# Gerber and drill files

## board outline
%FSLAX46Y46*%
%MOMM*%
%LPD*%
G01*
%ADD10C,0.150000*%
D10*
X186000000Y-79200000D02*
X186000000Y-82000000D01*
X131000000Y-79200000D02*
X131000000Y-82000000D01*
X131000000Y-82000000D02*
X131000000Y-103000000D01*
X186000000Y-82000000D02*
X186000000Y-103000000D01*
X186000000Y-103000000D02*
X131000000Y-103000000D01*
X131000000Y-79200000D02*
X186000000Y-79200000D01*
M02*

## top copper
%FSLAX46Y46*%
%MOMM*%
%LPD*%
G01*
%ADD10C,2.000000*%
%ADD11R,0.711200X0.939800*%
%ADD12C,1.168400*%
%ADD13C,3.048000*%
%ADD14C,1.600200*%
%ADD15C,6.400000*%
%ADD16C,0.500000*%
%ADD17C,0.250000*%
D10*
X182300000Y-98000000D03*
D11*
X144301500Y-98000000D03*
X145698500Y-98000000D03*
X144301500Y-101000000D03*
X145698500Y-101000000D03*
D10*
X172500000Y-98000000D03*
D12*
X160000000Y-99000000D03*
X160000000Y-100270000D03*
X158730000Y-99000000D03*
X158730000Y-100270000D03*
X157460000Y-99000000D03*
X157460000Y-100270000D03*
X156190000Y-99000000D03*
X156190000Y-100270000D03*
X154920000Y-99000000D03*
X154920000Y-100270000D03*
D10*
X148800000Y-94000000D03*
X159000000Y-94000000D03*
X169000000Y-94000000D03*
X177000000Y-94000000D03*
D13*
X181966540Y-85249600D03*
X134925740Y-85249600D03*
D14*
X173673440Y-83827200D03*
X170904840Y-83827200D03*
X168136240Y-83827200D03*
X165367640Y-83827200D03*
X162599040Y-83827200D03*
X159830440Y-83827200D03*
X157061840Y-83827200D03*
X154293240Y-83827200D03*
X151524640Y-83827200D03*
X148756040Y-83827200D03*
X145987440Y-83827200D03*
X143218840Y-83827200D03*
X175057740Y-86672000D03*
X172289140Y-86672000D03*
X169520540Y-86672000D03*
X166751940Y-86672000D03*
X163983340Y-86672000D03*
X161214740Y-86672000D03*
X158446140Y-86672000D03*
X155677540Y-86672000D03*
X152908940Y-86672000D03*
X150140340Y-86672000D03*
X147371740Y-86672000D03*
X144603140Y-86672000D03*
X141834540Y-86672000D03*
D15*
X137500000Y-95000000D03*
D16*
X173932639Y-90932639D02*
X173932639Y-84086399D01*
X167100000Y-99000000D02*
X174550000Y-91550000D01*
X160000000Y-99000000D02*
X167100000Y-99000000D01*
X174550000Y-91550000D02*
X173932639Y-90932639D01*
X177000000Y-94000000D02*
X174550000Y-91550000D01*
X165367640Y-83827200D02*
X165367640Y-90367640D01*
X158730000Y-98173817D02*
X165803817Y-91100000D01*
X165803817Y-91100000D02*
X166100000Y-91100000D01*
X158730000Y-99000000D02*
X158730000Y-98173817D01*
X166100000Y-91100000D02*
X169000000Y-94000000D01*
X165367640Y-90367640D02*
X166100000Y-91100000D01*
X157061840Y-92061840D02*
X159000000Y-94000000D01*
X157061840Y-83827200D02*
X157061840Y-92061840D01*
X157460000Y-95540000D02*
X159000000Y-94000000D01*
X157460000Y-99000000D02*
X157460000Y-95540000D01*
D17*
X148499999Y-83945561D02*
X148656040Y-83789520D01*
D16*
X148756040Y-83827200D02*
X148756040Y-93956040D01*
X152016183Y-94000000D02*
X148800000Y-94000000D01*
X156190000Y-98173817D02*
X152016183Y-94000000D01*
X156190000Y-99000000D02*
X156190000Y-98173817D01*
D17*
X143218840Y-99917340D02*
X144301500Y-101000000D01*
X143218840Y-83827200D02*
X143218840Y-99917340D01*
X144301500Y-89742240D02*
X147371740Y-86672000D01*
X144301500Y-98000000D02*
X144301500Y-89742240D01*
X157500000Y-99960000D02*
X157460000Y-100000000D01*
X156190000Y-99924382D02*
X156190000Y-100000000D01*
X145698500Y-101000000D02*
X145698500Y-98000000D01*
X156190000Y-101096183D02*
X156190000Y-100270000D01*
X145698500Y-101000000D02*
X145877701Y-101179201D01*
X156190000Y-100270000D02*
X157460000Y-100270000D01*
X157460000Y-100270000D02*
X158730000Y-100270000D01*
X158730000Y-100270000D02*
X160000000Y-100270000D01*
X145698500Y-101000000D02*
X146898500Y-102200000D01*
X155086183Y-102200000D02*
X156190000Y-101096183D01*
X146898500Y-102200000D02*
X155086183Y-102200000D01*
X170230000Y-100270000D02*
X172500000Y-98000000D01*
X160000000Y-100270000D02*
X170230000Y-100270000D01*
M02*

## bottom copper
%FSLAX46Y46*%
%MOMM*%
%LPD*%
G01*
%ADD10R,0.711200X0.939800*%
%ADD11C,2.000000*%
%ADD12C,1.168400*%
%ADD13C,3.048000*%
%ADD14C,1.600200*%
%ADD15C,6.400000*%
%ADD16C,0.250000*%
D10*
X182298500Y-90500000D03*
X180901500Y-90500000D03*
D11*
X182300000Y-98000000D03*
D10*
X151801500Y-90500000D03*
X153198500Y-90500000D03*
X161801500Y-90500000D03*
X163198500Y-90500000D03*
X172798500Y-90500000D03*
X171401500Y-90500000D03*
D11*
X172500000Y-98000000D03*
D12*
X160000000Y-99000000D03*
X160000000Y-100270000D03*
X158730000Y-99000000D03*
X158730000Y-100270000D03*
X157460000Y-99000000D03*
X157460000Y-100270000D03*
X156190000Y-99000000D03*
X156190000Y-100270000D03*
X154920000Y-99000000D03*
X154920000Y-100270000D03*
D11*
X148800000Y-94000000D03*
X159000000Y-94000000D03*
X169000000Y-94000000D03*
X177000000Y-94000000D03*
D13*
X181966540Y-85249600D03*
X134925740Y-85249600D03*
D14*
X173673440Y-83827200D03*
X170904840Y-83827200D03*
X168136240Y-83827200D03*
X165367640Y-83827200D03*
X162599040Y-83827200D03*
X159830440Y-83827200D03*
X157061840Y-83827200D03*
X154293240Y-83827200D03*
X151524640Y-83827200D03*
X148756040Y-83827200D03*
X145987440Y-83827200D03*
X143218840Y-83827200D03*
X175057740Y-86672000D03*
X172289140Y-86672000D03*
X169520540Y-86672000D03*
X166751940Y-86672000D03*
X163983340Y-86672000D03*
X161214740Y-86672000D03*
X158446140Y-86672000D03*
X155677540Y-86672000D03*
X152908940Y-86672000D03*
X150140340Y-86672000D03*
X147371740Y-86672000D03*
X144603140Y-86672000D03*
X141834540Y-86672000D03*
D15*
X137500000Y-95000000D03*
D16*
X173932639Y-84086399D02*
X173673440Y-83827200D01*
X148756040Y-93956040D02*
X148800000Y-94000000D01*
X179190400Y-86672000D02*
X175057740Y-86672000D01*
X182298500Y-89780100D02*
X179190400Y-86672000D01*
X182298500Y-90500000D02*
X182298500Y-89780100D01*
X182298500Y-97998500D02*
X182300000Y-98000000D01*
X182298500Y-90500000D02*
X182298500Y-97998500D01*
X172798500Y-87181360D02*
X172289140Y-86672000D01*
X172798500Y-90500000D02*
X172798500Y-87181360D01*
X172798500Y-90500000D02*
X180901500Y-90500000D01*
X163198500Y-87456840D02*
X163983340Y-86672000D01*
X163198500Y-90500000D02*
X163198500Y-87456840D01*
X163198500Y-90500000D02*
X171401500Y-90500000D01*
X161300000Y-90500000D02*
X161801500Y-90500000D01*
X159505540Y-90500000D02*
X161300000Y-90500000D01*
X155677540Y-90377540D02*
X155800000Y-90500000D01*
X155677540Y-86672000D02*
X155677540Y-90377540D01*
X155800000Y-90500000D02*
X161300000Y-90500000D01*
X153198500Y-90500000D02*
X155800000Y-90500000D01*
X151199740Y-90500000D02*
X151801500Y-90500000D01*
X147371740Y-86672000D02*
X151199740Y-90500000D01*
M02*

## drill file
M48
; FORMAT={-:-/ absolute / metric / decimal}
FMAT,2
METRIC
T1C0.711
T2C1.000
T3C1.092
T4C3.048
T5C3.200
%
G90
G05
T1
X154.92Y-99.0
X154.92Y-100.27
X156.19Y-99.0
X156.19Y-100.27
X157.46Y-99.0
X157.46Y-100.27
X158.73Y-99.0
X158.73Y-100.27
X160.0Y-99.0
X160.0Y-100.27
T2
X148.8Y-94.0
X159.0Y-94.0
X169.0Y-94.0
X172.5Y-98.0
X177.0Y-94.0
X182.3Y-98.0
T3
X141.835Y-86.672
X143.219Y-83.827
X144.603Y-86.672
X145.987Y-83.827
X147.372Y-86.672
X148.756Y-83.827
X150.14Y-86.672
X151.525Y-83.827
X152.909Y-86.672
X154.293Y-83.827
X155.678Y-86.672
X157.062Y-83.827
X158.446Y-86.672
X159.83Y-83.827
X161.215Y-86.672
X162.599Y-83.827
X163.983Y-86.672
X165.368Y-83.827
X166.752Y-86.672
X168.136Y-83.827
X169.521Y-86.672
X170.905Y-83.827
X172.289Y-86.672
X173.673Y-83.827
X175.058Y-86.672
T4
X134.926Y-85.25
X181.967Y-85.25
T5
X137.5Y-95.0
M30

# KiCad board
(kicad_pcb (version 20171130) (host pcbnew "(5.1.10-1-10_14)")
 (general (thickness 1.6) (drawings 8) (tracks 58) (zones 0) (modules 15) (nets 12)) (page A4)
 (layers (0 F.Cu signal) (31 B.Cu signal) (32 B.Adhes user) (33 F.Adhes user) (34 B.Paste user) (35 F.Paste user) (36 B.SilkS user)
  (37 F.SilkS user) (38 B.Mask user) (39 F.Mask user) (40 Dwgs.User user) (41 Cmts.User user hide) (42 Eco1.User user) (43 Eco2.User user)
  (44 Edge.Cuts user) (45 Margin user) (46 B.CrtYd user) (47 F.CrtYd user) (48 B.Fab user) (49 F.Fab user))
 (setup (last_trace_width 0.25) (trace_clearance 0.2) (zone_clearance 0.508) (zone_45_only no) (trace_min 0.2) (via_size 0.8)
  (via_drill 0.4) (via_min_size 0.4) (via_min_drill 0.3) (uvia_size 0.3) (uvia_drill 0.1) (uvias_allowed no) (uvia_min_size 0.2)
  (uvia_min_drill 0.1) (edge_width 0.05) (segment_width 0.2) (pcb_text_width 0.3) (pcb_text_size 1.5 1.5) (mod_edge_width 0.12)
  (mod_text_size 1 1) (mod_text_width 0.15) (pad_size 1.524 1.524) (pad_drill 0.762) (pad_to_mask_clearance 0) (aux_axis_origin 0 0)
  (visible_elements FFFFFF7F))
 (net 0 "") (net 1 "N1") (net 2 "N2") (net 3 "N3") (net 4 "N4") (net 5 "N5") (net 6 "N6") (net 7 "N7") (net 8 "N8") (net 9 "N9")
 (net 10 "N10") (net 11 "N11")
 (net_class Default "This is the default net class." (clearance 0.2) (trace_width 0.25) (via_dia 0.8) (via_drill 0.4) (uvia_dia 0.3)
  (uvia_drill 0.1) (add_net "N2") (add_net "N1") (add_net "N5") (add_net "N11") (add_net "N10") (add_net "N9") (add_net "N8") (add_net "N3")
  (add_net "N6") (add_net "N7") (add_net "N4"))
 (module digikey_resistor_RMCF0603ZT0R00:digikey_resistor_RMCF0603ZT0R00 (layer B.Cu) (at 181.6 90.5)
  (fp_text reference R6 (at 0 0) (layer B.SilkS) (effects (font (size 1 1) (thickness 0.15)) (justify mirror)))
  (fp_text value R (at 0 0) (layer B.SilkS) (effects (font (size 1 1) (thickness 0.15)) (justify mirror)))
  (pad 2 smd rect (at 0.6985 0) (size 0.7112 0.9398) (layers B.Cu B.Paste B.Mask) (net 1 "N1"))
  (pad 1 smd rect (at -0.6985 0) (size 0.7112 0.9398) (layers B.Cu B.Paste B.Mask) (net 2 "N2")))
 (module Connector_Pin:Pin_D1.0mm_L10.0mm (layer F.Cu) (at 182.3 98)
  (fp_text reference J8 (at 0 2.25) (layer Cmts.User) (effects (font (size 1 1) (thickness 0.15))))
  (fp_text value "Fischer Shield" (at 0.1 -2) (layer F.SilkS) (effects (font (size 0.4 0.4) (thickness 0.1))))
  (pad 1 thru_hole circle (at 0 0) (size 2 2) (drill 1) (layers *.Cu *.Mask) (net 1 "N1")))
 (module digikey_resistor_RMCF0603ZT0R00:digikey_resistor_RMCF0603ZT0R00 (layer F.Cu) (at 145 98 180)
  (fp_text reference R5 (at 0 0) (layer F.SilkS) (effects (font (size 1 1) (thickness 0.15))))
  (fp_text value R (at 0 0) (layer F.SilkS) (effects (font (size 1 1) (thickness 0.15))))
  (pad 2 smd rect (at 0.6985 0 180) (size 0.7112 0.9398) (layers F.Cu F.Paste F.Mask) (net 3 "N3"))
  (pad 1 smd rect (at -0.6985 0 180) (size 0.7112 0.9398) (layers F.Cu F.Paste F.Mask) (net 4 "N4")))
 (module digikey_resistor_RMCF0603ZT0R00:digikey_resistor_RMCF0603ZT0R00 (layer F.Cu) (at 145 101 180)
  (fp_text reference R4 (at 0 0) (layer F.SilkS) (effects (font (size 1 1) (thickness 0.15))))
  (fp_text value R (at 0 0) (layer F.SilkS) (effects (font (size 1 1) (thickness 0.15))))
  (pad 2 smd rect (at 0.6985 0 180) (size 0.7112 0.9398) (layers F.Cu F.Paste F.Mask) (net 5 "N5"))
  (pad 1 smd rect (at -0.6985 0 180) (size 0.7112 0.9398) (layers F.Cu F.Paste F.Mask) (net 4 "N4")))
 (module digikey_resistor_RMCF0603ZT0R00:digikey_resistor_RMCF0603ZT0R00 (layer B.Cu) (at 152.5 90.5 180)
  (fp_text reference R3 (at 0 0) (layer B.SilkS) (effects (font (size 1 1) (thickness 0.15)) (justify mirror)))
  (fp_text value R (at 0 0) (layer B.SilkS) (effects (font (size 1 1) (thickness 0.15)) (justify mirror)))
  (pad 2 smd rect (at 0.6985 0 180) (size 0.7112 0.9398) (layers B.Cu B.Paste B.Mask) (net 3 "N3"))
  (pad 1 smd rect (at -0.6985 0 180) (size 0.7112 0.9398) (layers B.Cu B.Paste B.Mask) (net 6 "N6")))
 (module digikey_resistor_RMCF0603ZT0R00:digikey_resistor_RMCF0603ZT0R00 (layer B.Cu) (at 162.5 90.5 180)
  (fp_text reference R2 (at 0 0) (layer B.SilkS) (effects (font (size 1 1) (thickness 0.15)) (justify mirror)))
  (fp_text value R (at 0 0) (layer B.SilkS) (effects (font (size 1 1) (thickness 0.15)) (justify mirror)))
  (pad 2 smd rect (at 0.6985 0 180) (size 0.7112 0.9398) (layers B.Cu B.Paste B.Mask) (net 6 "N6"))
  (pad 1 smd rect (at -0.6985 0 180) (size 0.7112 0.9398) (layers B.Cu B.Paste B.Mask) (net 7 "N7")))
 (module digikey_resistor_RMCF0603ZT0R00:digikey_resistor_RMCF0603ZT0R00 (layer B.Cu) (at 172.1 90.5)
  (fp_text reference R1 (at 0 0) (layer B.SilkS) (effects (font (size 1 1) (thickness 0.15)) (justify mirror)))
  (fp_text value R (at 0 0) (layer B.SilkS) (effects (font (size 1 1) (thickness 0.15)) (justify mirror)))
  (pad 2 smd rect (at 0.6985 0) (size 0.7112 0.9398) (layers B.Cu B.Paste B.Mask) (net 2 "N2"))
  (pad 1 smd rect (at -0.6985 0) (size 0.7112 0.9398) (layers B.Cu B.Paste B.Mask) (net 7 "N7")))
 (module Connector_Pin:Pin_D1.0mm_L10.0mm (layer F.Cu) (at 172.5 98)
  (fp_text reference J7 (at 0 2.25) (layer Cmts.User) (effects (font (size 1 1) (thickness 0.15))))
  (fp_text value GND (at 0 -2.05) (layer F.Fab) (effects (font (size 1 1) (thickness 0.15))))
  (pad 1 thru_hole circle (at 0 0) (size 2 2) (drill 1) (layers *.Cu *.Mask) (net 4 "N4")))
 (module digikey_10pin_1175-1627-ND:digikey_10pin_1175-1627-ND (layer F.Cu) (at 160 99 180)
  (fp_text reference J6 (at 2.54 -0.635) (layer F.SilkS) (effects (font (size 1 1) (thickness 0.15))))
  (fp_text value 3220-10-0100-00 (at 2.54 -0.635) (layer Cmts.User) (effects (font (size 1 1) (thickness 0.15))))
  (pad 1 thru_hole circle (at 0 0 180) (size 1.1684 1.1684) (drill 0.7112) (layers *.Cu *.Mask) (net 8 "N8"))
  (pad 2 thru_hole circle (at 0 -1.27 180) (size 1.1684 1.1684) (drill 0.7112) (layers *.Cu *.Mask) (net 4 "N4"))
  (pad 3 thru_hole circle (at 1.27 0 180) (size 1.1684 1.1684) (drill 0.7112) (layers *.Cu *.Mask) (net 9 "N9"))
  (pad 4 thru_hole circle (at 1.27 -1.27 180) (size 1.1684 1.1684) (drill 0.7112) (layers *.Cu *.Mask) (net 4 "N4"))
  (pad 5 thru_hole circle (at 2.54 0 180) (size 1.1684 1.1684) (drill 0.7112) (layers *.Cu *.Mask) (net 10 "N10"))
  (pad 6 thru_hole circle (at 2.54 -1.27 180) (size 1.1684 1.1684) (drill 0.7112) (layers *.Cu *.Mask) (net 4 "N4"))
  (pad 7 thru_hole circle (at 3.81 0 180) (size 1.1684 1.1684) (drill 0.7112) (layers *.Cu *.Mask) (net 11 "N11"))
  (pad 8 thru_hole circle (at 3.81 -1.27 180) (size 1.1684 1.1684) (drill 0.7112) (layers *.Cu *.Mask) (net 4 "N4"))
  (pad 9 thru_hole circle (at 5.08 0 180) (size 1.1684 1.1684) (drill 0.7112) (layers *.Cu *.Mask))
  (pad 10 thru_hole circle (at 5.08 -1.27 180) (size 1.1684 1.1684) (drill 0.7112) (layers *.Cu *.Mask)))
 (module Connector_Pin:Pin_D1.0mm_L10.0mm (layer F.Cu) (at 148.8 94)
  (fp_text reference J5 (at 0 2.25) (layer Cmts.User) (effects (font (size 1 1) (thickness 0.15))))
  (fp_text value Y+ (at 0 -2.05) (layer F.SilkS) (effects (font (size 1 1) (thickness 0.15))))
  (pad 1 thru_hole circle (at 0 0) (size 2 2) (drill 1) (layers *.Cu *.Mask) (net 11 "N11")))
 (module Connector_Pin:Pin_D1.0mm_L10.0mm (layer F.Cu) (at 159 94)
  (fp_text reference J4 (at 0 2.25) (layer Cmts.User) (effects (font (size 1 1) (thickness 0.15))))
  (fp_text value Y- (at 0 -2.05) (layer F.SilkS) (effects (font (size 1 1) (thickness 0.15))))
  (pad 1 thru_hole circle (at 0 0) (size 2 2) (drill 1) (layers *.Cu *.Mask) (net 10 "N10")))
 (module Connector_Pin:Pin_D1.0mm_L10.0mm (layer F.Cu) (at 169 94)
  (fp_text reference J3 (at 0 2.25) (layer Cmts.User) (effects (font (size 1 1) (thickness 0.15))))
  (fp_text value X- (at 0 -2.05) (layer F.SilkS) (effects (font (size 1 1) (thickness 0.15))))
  (pad 1 thru_hole circle (at 0 0) (size 2 2) (drill 1) (layers *.Cu *.Mask) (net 9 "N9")))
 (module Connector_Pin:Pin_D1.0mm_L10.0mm (layer F.Cu) (at 177 94)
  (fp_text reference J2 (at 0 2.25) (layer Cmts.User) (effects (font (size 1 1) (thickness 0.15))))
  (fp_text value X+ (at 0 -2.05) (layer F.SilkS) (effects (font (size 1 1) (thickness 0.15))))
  (pad 1 thru_hole circle (at 0 0) (size 2 2) (drill 1) (layers *.Cu *.Mask) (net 8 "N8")))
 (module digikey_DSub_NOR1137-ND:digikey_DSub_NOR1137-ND (layer F.Cu) (at 158.44614 75.75)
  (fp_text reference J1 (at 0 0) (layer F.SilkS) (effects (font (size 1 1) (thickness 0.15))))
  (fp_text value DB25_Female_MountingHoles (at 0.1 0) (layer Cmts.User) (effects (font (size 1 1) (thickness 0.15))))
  (pad 27 thru_hole circle (at 23.5204 9.4996) (size 3.048 3.048) (drill 3.048) (layers *.Cu *.Mask))
  (pad 26 thru_hole circle (at -23.5204 9.4996) (size 3.048 3.048) (drill 3.048) (layers *.Cu *.Mask))
  (pad 25 thru_hole circle (at 15.2273 8.0772) (size 1.6002 1.6002) (drill 1.0922) (layers *.Cu *.Mask) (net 8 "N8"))
  (pad 24 thru_hole circle (at 12.4587 8.0772) (size 1.6002 1.6002) (drill 1.0922) (layers *.Cu *.Mask))
  (pad 23 thru_hole circle (at 9.6901 8.0772) (size 1.6002 1.6002) (drill 1.0922) (layers *.Cu *.Mask))
  (pad 22 thru_hole circle (at 6.9215 8.0772) (size 1.6002 1.6002) (drill 1.0922) (layers *.Cu *.Mask) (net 9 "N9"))
  (pad 21 thru_hole circle (at 4.1529 8.0772) (size 1.6002 1.6002) (drill 1.0922) (layers *.Cu *.Mask))
  (pad 20 thru_hole circle (at 1.3843 8.0772) (size 1.6002 1.6002) (drill 1.0922) (layers *.Cu *.Mask))
  (pad 19 thru_hole circle (at -1.3843 8.0772) (size 1.6002 1.6002) (drill 1.0922) (layers *.Cu *.Mask) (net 10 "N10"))
  (pad 18 thru_hole circle (at -4.1529 8.0772) (size 1.6002 1.6002) (drill 1.0922) (layers *.Cu *.Mask))
  (pad 17 thru_hole circle (at -6.9215 8.0772) (size 1.6002 1.6002) (drill 1.0922) (layers *.Cu *.Mask))
  (pad 16 thru_hole circle (at -9.6901 8.0772) (size 1.6002 1.6002) (drill 1.0922) (layers *.Cu *.Mask) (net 11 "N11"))
  (pad 15 thru_hole circle (at -12.4587 8.0772) (size 1.6002 1.6002) (drill 1.0922) (layers *.Cu *.Mask))
  (pad 14 thru_hole circle (at -15.2273 8.0772) (size 1.6002 1.6002) (drill 1.0922) (layers *.Cu *.Mask) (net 5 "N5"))
  (pad 13 thru_hole circle (at 16.6116 10.922) (size 1.6002 1.6002) (drill 1.0922) (layers *.Cu *.Mask) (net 1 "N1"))
  (pad 12 thru_hole circle (at 13.843 10.922) (size 1.6002 1.6002) (drill 1.0922) (layers *.Cu *.Mask) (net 2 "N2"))
  (pad 11 thru_hole circle (at 11.0744 10.922) (size 1.6002 1.6002) (drill 1.0922) (layers *.Cu *.Mask))
  (pad 10 thru_hole circle (at 8.3058 10.922) (size 1.6002 1.6002) (drill 1.0922) (layers *.Cu *.Mask))
  (pad 9 thru_hole circle (at 5.5372 10.922) (size 1.6002 1.6002) (drill 1.0922) (layers *.Cu *.Mask) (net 7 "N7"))
  (pad 8 thru_hole circle (at 2.7686 10.922) (size 1.6002 1.6002) (drill 1.0922) (layers *.Cu *.Mask))
  (pad 7 thru_hole circle (at 0 10.922) (size 1.6002 1.6002) (drill 1.0922) (layers *.Cu *.Mask))
  (pad 6 thru_hole circle (at -2.7686 10.922) (size 1.6002 1.6002) (drill 1.0922) (layers *.Cu *.Mask) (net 6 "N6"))
  (pad 5 thru_hole circle (at -5.5372 10.922) (size 1.6002 1.6002) (drill 1.0922) (layers *.Cu *.Mask))
  (pad 4 thru_hole circle (at -8.3058 10.922) (size 1.6002 1.6002) (drill 1.0922) (layers *.Cu *.Mask))
  (pad 3 thru_hole circle (at -11.0744 10.922) (size 1.6002 1.6002) (drill 1.0922) (layers *.Cu *.Mask) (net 3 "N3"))
  (pad 2 thru_hole circle (at -13.843 10.922) (size 1.6002 1.6002) (drill 1.0922) (layers *.Cu *.Mask))
  (pad 1 thru_hole circle (at -16.6116 10.922) (size 1.6002 1.6002) (drill 1.0922) (layers *.Cu *.Mask)))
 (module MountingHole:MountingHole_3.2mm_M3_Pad (layer F.Cu) (at 137.5 95)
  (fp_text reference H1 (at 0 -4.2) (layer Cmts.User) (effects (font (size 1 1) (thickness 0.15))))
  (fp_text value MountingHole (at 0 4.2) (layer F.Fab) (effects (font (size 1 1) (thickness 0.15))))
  (pad 1 thru_hole circle (at 0 0) (size 6.4 6.4) (drill 3.2) (layers *.Cu *.Mask)))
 (gr_line (start 186 79.2) (end 186 82) (layer Edge.Cuts) (width 0.15))
 (gr_line (start 131 79.2) (end 131 82) (layer Edge.Cuts) (width 0.15))
 (gr_line (start 131 82) (end 131 103) (layer Edge.Cuts) (width 0.15))
 (gr_line (start 186 82) (end 186 103) (layer Edge.Cuts) (width 0.15))
 (gr_line (start 186 103) (end 131 103) (layer Edge.Cuts) (width 0.15))
 (gr_line (start 131 79.2) (end 186 79.2) (layer Edge.Cuts) (width 0.15))
 (segment (start 173.932639 84.086399) (end 173.67344 83.8272) (width 0.25) (layer B.Cu) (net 8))
 (segment (start 173.932639 90.932639) (end 173.932639 84.086399) (width 0.5) (layer F.Cu) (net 8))
 (segment (start 167.1 99) (end 174.55 91.55) (width 0.5) (layer F.Cu) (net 8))
 (segment (start 160 99) (end 167.1 99) (width 0.5) (layer F.Cu) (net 8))
 (segment (start 174.55 91.55) (end 173.932639 90.932639) (width 0.5) (layer F.Cu) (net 8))
 (segment (start 177 94) (end 174.55 91.55) (width 0.5) (layer F.Cu) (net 8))
 (segment (start 165.36764 83.8272) (end 165.36764 90.36764) (width 0.5) (layer F.Cu) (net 9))
 (segment (start 158.73 98.173817) (end 165.803817 91.1) (width 0.5) (layer F.Cu) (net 9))
 (segment (start 165.803817 91.1) (end 166.1 91.1) (width 0.5) (layer F.Cu) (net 9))
 (segment (start 158.73 99) (end 158.73 98.173817) (width 0.5) (layer F.Cu) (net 9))
 (segment (start 166.1 91.1) (end 169 94) (width 0.5) (layer F.Cu) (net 9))
 (segment (start 165.36764 90.36764) (end 166.1 91.1) (width 0.5) (layer F.Cu) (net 9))
 (segment (start 157.06184 92.06184) (end 159 94) (width 0.5) (layer F.Cu) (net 10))
 (segment (start 157.06184 83.8272) (end 157.06184 92.06184) (width 0.5) (layer F.Cu) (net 10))
 (segment (start 157.46 95.54) (end 159 94) (width 0.5) (layer F.Cu) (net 10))
 (segment (start 157.46 99) (end 157.46 95.54) (width 0.5) (layer F.Cu) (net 10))
 (segment (start 148.499999 83.945561) (end 148.65604 83.78952) (width 0.25) (layer F.Cu) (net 11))
 (segment (start 148.75604 93.95604) (end 148.8 94) (width 0.25) (layer B.Cu) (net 11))
 (segment (start 148.75604 83.8272) (end 148.75604 93.95604) (width 0.5) (layer F.Cu) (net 11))
 (segment (start 152.016183 94) (end 148.8 94) (width 0.5) (layer F.Cu) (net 11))
 (segment (start 156.19 98.173817) (end 152.016183 94) (width 0.5) (layer F.Cu) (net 11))
 (segment (start 156.19 99) (end 156.19 98.173817) (width 0.5) (layer F.Cu) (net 11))
 (segment (start 143.21884 99.91734) (end 144.3015 101) (width 0.25) (layer F.Cu) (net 5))
 (segment (start 143.21884 83.8272) (end 143.21884 99.91734) (width 0.25) (layer F.Cu) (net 5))
 (segment (start 179.1904 86.672) (end 175.05774 86.672) (width 0.25) (layer B.Cu) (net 1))
 (segment (start 182.2985 89.7801) (end 179.1904 86.672) (width 0.25) (layer B.Cu) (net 1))
 (segment (start 182.2985 90.5) (end 182.2985 89.7801) (width 0.25) (layer B.Cu) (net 1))
 (segment (start 182.2985 97.9985) (end 182.3 98) (width 0.25) (layer B.Cu) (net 1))
 (segment (start 182.2985 90.5) (end 182.2985 97.9985) (width 0.25) (layer B.Cu) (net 1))
 (segment (start 172.7985 87.18136) (end 172.28914 86.672) (width 0.25) (layer B.Cu) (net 2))
 (segment (start 172.7985 90.5) (end 172.7985 87.18136) (width 0.25) (layer B.Cu) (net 2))
 (segment (start 172.7985 90.5) (end 180.9015 90.5) (width 0.25) (layer B.Cu) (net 2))
 (segment (start 163.1985 87.45684) (end 163.98334 86.672) (width 0.25) (layer B.Cu) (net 7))
 (segment (start 163.1985 90.5) (end 163.1985 87.45684) (width 0.25) (layer B.Cu) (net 7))
 (segment (start 163.1985 90.5) (end 171.4015 90.5) (width 0.25) (layer B.Cu) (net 7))
 (segment (start 161.3 90.5) (end 161.8015 90.5) (width 0.25) (layer B.Cu) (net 6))
 (segment (start 159.50554 90.5) (end 161.3 90.5) (width 0.25) (layer B.Cu) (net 6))
 (segment (start 155.67754 90.37754) (end 155.8 90.5) (width 0.25) (layer B.Cu) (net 6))
 (segment (start 155.67754 86.672) (end 155.67754 90.37754) (width 0.25) (layer B.Cu) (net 6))
 (segment (start 155.8 90.5) (end 161.3 90.5) (width 0.25) (layer B.Cu) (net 6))
 (segment (start 153.1985 90.5) (end 155.8 90.5) (width 0.25) (layer B.Cu) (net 6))
 (segment (start 144.3015 89.74224) (end 147.37174 86.672) (width 0.25) (layer F.Cu) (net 3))
 (segment (start 144.3015 98) (end 144.3015 89.74224) (width 0.25) (layer F.Cu) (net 3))
 (segment (start 151.19974 90.5) (end 151.8015 90.5) (width 0.25) (layer B.Cu) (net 3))
 (segment (start 147.37174 86.672) (end 151.19974 90.5) (width 0.25) (layer B.Cu) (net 3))
 (segment (start 157.5 99.96) (end 157.46 100) (width 0.25) (layer F.Cu) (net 4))
 (segment (start 156.19 99.924382) (end 156.19 100) (width 0.25) (layer F.Cu) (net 4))
 (segment (start 145.6985 101) (end 145.6985 98) (width 0.25) (layer F.Cu) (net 4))
 (segment (start 156.19 101.096183) (end 156.19 100.27) (width 0.25) (layer F.Cu) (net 4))
 (segment (start 145.6985 101) (end 145.877701 101.179201) (width 0.25) (layer F.Cu) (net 4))
 (segment (start 156.19 100.27) (end 157.46 100.27) (width 0.25) (layer F.Cu) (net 4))
 (segment (start 157.46 100.27) (end 158.73 100.27) (width 0.25) (layer F.Cu) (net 4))
 (segment (start 158.73 100.27) (end 160 100.27) (width 0.25) (layer F.Cu) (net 4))
 (segment (start 145.6985 101) (end 146.8985 102.2) (width 0.25) (layer F.Cu) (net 4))
 (segment (start 155.086183 102.2) (end 156.19 101.096183) (width 0.25) (layer F.Cu) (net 4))
 (segment (start 146.8985 102.2) (end 155.086183 102.2) (width 0.25) (layer F.Cu) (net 4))
 (segment (start 170.23 100.27) (end 172.5 98) (width 0.25) (layer F.Cu) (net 4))
 (segment (start 160 100.27) (end 170.23 100.27) (width 0.25) (layer F.Cu) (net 4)))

